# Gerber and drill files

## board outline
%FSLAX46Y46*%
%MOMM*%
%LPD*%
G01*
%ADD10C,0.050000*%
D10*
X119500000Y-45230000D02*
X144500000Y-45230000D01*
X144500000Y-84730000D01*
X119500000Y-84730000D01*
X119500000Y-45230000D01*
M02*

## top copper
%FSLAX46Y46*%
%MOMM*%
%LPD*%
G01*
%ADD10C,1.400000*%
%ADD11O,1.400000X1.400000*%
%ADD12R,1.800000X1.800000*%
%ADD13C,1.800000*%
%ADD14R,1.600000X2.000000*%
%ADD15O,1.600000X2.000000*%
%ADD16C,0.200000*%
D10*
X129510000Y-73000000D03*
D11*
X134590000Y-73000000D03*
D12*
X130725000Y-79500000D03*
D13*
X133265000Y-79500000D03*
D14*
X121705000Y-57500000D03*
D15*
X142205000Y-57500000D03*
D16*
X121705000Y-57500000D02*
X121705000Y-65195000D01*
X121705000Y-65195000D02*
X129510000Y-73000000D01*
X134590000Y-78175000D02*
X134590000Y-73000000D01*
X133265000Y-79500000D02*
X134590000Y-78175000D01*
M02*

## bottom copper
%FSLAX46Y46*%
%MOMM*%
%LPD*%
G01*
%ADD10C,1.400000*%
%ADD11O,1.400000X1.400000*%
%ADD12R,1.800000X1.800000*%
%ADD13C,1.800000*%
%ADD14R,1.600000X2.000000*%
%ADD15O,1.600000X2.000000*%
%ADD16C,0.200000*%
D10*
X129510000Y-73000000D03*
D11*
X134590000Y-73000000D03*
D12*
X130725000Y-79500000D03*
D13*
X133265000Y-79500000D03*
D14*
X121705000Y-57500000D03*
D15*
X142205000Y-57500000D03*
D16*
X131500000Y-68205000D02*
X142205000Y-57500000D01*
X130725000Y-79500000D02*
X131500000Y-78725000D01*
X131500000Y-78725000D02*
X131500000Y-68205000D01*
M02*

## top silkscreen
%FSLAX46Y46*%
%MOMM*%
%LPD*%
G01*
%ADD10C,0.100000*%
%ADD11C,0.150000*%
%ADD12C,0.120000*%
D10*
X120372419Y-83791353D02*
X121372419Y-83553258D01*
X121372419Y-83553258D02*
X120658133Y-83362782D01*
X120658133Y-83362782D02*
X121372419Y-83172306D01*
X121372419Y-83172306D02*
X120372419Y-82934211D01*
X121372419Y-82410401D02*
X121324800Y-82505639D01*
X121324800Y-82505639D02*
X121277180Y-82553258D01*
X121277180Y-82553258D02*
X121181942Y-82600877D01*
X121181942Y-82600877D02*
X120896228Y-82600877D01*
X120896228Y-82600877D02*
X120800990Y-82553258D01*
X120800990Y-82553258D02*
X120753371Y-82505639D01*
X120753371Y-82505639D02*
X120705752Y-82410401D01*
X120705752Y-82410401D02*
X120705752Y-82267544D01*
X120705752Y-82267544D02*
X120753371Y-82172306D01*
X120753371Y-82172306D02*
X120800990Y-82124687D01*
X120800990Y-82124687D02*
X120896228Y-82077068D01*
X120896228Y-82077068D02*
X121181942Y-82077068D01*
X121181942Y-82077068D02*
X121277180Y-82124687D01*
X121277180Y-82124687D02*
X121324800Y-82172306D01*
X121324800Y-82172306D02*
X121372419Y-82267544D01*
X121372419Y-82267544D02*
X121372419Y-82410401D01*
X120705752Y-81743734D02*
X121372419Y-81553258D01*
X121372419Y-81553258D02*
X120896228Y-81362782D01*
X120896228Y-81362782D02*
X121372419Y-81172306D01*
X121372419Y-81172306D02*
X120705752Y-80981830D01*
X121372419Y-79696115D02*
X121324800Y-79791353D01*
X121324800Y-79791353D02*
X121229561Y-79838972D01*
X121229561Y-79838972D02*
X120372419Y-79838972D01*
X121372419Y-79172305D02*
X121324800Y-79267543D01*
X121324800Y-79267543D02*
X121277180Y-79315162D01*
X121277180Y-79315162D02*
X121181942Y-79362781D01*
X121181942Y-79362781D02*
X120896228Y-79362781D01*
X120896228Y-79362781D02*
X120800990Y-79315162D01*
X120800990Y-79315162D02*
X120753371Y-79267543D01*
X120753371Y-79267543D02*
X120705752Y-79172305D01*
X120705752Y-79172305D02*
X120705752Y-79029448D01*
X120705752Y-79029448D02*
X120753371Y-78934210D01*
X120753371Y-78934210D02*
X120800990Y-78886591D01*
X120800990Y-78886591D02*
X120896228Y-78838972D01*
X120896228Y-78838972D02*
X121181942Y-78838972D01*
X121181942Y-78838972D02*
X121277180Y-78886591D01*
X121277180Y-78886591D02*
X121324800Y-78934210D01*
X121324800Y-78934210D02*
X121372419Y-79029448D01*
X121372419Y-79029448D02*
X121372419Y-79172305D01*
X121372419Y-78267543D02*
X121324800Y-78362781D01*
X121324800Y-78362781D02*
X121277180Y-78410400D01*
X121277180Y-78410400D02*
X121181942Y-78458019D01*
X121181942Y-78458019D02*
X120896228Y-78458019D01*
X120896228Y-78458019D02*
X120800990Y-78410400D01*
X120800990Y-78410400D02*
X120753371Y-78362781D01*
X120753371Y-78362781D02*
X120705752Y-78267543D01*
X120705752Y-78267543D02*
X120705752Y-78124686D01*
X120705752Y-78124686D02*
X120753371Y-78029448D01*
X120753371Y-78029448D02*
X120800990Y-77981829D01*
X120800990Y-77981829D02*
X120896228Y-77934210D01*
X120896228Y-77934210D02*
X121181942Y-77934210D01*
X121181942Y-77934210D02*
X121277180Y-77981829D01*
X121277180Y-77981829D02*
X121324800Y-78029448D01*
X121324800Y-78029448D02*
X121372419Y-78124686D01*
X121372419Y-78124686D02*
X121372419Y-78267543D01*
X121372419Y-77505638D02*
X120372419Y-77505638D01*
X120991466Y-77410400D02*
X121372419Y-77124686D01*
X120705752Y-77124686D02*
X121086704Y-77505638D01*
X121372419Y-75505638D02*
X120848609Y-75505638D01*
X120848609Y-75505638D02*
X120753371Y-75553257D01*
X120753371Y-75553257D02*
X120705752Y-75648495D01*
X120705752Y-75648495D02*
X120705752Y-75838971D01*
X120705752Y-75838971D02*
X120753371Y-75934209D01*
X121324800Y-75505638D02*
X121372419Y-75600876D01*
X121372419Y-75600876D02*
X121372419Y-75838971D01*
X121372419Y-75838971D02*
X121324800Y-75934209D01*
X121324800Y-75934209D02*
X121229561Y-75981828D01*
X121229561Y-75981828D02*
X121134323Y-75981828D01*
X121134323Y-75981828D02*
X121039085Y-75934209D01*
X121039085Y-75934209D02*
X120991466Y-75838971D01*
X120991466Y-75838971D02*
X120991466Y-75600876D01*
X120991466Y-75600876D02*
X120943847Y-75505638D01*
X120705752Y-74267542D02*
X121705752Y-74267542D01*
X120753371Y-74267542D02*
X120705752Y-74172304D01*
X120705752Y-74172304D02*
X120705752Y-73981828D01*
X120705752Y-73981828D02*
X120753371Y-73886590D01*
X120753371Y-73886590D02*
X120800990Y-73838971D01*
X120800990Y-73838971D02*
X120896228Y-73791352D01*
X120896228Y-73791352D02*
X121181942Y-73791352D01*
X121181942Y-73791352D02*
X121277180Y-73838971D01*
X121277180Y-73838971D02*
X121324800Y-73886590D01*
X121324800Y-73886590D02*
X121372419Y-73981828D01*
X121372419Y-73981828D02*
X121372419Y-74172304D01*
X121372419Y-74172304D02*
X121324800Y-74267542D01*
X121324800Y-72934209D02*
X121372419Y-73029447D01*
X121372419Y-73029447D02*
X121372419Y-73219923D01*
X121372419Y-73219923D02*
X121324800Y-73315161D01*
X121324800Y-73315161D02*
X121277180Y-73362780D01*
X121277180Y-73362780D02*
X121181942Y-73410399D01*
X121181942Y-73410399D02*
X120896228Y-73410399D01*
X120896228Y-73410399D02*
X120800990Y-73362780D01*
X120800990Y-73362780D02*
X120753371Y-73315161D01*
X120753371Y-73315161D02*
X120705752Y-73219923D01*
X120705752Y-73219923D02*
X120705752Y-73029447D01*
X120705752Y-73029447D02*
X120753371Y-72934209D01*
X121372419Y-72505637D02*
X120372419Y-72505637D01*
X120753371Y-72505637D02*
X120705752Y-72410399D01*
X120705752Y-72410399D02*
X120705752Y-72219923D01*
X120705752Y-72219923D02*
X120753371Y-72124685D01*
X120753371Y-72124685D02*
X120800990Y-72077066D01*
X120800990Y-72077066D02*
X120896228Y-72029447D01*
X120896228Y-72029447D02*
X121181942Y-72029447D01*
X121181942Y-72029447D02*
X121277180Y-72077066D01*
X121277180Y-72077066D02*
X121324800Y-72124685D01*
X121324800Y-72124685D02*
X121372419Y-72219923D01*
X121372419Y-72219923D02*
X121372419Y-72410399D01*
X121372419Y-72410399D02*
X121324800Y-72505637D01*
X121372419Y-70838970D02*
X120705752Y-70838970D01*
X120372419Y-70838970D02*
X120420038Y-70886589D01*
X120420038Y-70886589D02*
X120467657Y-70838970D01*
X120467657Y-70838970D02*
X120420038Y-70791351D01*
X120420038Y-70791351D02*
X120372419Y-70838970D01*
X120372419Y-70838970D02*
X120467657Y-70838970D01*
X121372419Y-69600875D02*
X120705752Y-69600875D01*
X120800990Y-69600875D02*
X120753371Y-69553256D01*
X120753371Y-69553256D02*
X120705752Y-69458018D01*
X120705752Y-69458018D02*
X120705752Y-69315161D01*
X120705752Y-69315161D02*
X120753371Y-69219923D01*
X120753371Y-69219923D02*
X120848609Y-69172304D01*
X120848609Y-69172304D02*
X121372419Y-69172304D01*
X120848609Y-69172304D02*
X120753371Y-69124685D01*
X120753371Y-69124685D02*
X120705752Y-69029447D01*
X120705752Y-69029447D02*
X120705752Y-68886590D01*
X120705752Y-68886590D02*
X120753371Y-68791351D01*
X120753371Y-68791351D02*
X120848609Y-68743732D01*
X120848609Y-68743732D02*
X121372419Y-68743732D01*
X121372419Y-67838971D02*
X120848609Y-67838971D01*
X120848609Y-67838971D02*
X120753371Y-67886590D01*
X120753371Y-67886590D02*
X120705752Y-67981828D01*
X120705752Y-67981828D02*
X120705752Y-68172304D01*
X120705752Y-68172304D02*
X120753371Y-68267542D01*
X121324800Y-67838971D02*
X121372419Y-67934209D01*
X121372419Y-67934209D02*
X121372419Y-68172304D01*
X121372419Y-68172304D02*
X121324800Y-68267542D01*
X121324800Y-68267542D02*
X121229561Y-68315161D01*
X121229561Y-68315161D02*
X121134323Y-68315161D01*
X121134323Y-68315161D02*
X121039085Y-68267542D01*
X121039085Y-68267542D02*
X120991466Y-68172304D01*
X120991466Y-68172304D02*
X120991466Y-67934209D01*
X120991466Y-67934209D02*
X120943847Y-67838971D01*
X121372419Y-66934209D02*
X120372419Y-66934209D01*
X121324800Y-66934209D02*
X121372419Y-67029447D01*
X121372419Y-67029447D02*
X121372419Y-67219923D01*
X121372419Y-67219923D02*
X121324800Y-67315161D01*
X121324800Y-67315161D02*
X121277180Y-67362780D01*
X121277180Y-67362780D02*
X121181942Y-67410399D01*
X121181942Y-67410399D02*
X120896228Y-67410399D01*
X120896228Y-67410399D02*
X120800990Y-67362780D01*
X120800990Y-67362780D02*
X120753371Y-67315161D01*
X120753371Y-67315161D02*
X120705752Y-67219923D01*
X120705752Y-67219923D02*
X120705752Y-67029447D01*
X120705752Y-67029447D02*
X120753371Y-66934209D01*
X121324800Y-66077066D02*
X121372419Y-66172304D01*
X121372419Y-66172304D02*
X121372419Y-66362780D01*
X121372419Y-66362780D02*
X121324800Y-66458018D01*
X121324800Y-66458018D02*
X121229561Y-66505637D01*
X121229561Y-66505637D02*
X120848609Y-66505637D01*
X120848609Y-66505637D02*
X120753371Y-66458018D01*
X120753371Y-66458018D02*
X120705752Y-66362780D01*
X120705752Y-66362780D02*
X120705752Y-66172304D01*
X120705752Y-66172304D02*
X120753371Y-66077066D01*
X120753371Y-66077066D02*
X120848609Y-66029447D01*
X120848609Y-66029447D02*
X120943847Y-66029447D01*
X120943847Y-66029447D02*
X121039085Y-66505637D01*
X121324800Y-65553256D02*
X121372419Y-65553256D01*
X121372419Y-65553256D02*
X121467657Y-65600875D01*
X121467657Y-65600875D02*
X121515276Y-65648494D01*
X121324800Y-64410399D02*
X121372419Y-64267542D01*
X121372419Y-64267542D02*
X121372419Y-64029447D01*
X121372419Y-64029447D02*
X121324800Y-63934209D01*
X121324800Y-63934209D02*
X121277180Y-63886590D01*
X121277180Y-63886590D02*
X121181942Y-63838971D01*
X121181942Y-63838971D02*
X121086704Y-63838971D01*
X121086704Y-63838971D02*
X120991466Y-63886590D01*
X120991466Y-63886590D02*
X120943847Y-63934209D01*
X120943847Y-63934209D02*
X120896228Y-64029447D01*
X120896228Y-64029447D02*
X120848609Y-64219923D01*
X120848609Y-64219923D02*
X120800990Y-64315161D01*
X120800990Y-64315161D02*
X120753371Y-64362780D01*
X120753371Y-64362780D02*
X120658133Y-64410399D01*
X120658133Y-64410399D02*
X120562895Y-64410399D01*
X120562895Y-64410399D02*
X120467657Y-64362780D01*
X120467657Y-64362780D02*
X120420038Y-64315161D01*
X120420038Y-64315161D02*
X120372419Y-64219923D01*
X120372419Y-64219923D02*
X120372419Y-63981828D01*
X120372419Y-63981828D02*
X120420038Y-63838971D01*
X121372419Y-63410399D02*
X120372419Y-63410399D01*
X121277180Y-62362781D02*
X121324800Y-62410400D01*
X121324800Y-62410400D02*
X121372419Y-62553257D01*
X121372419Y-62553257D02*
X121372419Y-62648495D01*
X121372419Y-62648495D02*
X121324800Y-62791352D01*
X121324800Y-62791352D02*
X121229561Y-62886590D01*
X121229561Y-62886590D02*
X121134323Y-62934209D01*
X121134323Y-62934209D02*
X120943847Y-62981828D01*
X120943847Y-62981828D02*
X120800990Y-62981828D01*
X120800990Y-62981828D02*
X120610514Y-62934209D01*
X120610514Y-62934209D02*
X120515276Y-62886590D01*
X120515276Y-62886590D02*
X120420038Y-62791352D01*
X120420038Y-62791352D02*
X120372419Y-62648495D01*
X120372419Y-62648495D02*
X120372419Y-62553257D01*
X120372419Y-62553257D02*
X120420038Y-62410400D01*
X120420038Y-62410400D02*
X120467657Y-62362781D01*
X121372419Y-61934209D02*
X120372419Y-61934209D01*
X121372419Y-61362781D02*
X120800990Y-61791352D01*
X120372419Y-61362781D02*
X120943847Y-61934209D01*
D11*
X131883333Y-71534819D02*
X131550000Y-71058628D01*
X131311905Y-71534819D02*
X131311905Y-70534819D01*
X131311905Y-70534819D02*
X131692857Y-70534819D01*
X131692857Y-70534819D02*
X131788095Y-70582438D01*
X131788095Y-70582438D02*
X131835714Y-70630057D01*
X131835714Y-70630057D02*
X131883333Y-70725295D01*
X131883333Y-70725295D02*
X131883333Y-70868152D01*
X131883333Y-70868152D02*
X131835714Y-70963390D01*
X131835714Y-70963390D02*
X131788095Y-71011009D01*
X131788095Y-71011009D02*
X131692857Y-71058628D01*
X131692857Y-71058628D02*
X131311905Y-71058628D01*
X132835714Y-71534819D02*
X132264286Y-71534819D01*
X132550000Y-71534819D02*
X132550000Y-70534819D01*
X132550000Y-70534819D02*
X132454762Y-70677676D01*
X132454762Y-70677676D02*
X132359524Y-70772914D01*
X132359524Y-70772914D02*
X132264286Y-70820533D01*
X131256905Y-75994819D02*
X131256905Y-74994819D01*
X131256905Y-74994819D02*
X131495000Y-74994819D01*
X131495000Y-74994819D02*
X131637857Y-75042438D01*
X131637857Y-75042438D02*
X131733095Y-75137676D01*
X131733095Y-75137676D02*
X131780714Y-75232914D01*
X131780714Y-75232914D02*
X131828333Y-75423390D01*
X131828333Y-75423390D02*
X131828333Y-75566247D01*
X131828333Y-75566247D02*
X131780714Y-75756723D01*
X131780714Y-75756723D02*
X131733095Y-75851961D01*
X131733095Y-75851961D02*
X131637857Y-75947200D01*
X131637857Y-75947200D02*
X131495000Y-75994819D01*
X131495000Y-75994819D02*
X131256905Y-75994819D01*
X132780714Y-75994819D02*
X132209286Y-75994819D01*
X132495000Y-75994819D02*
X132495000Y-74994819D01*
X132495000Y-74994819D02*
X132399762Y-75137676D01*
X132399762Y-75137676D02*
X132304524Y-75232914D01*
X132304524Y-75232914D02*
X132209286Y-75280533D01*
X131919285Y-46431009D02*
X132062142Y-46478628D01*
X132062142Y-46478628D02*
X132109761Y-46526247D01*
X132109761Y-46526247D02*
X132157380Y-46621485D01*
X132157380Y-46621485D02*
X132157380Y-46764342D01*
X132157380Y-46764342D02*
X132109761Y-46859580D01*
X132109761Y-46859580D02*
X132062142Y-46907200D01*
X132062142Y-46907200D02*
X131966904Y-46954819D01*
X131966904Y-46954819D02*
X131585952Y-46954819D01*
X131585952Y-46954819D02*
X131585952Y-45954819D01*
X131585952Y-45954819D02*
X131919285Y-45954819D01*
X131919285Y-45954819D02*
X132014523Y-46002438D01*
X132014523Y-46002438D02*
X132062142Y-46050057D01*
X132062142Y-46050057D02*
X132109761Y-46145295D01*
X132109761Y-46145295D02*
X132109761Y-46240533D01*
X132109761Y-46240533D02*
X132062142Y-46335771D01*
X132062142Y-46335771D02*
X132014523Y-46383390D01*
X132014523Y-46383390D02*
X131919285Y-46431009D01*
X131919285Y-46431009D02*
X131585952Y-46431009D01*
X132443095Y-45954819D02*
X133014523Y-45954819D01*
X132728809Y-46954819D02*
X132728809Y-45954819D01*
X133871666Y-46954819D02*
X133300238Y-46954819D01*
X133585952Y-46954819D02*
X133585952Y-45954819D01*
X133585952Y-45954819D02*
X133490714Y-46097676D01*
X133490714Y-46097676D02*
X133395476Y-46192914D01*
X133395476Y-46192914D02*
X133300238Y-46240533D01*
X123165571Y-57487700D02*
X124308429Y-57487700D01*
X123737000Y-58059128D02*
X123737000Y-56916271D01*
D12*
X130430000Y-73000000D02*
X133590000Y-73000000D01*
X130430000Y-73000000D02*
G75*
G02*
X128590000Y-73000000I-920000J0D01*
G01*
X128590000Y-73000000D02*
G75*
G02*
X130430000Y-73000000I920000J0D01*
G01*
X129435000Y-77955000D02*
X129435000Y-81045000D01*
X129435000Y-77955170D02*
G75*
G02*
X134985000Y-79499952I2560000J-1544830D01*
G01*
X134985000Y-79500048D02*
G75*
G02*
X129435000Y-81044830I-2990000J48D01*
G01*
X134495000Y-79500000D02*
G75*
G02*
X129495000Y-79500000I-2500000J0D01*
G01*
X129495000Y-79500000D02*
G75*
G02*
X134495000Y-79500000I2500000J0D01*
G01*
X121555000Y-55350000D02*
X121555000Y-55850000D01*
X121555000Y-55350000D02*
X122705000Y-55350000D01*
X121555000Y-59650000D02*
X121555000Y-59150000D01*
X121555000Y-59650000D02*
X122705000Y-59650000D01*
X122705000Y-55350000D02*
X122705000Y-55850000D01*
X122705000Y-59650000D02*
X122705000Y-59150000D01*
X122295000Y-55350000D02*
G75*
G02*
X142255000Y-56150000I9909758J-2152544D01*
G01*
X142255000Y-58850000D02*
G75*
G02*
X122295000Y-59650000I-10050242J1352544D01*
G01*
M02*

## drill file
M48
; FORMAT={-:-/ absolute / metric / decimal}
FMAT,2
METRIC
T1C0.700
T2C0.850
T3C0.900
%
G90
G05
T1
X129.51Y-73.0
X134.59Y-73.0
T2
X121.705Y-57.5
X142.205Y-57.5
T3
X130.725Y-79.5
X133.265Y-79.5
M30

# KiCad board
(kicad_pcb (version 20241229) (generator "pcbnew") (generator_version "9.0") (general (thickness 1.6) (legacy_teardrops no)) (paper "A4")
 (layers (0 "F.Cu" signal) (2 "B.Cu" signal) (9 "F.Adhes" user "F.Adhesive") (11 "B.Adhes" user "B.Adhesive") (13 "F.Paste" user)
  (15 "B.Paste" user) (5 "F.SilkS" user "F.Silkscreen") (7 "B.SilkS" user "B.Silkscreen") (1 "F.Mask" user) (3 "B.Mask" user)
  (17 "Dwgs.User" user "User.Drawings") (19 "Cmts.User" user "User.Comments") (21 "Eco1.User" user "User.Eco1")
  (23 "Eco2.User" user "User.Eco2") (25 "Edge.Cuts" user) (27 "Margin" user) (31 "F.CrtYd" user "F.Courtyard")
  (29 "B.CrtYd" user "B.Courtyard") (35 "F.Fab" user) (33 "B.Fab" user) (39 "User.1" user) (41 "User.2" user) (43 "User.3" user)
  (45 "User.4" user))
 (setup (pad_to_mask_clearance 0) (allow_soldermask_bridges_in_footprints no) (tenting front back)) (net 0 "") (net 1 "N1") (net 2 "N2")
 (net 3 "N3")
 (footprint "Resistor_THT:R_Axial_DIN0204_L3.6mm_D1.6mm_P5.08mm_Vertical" (layer "F.Cu") (at 129.51 73)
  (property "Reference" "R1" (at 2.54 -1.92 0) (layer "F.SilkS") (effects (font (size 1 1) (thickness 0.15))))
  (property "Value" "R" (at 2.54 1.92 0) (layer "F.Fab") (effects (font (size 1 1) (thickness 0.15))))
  (fp_line (start 0.92 0) (end 4.08 0) (stroke (width 0.12) (type solid)) (layer "F.SilkS"))
  (fp_circle (center 0 0) (end 0.92 0) (stroke (width 0.12) (type solid)) (fill no) (layer "F.SilkS"))
  (pad "1" thru_hole circle (at 0 0) (size 1.4 1.4) (drill 0.7) (layers "*.Cu" "*.Mask") (remove_unused_layers no) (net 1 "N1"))
  (pad "2" thru_hole oval (at 5.08 0) (size 1.4 1.4) (drill 0.7) (layers "*.Cu" "*.Mask") (remove_unused_layers no) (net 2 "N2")))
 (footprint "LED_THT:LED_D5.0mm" (layer "F.Cu") (at 130.725 79.5)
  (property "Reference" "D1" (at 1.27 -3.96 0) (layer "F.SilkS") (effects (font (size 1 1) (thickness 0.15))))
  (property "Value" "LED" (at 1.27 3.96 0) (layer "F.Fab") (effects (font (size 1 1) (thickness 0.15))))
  (fp_line (start -1.29 -1.545) (end -1.29 1.545) (stroke (width 0.12) (type solid)) (layer "F.SilkS"))
  (fp_arc (start -1.29 -1.54483) (mid 2.071756 -2.880501) (end 4.26 -0.000048) (stroke (width 0.12) (type solid)) (layer "F.SilkS"))
  (fp_arc (start 4.26 0.000048) (mid 2.071756 2.880501) (end -1.29 1.54483) (stroke (width 0.12) (type solid)) (layer "F.SilkS"))
  (fp_circle (center 1.27 0) (end 3.77 0) (stroke (width 0.12) (type solid)) (fill no) (layer "F.SilkS"))
  (pad "1" thru_hole rect (at 0 0) (size 1.8 1.8) (drill 0.9) (layers "*.Cu" "*.Mask") (remove_unused_layers no) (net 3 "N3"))
  (pad "2" thru_hole circle (at 2.54 0) (size 1.8 1.8) (drill 0.9) (layers "*.Cu" "*.Mask") (remove_unused_layers no) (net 2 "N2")))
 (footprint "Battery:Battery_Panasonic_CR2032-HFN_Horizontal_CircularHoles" (layer "F.Cu") (at 121.705 57.5)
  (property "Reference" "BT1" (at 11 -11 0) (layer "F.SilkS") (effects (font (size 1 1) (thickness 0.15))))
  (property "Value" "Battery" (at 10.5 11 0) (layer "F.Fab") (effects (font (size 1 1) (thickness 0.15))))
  (fp_line (start -0.15 -2.15) (end -0.15 -1.65) (stroke (width 0.12) (type default)) (layer "F.SilkS"))
  (fp_line (start -0.15 -2.15) (end 1 -2.15) (stroke (width 0.12) (type default)) (layer "F.SilkS"))
  (fp_line (start -0.15 2.15) (end -0.15 1.65) (stroke (width 0.12) (type default)) (layer "F.SilkS"))
  (fp_line (start -0.15 2.15) (end 1 2.15) (stroke (width 0.12) (type default)) (layer "F.SilkS"))
  (fp_line (start 1 -2.15) (end 1 -1.65) (stroke (width 0.12) (type default)) (layer "F.SilkS"))
  (fp_line (start 1 2.15) (end 1 1.65) (stroke (width 0.12) (type default)) (layer "F.SilkS"))
  (fp_arc (start 0.59 -2.15) (mid 10.91 -10.13) (end 20.55 -1.35) (stroke (width 0.12) (type default)) (layer "F.SilkS"))
  (fp_arc (start 20.55 1.35) (mid 10.91 10.13) (end 0.59 2.15) (stroke (width 0.12) (type default)) (layer "F.SilkS"))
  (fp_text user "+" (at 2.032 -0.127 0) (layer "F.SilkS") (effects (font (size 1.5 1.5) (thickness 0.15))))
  (pad "1" thru_hole rect (at 0 0) (size 1.6 2) (drill 0.85) (layers "*.Cu" "*.Mask") (remove_unused_layers no) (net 1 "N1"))
  (pad "2" thru_hole oval (at 20.5 0) (size 1.6 2) (drill 0.85) (layers "*.Cu" "*.Mask") (remove_unused_layers no) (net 3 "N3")))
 (gr_rect (start 119.5 45.23) (end 144.5 84.73) (stroke (width 0.05) (type default)) (fill no) (layer "Edge.Cuts"))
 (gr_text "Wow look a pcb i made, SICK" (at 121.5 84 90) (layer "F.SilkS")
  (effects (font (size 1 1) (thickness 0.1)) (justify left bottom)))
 (segment (start 121.705 57.5) (end 121.705 65.195) (width 0.2) (layer "F.Cu") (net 1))
 (segment (start 121.705 65.195) (end 129.51 73) (width 0.2) (layer "F.Cu") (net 1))
 (segment (start 131.5 68.205) (end 142.205 57.5) (width 0.2) (layer "B.Cu") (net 3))
 (segment (start 130.725 79.5) (end 131.5 78.725) (width 0.2) (layer "B.Cu") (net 3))
 (segment (start 131.5 78.725) (end 131.5 68.205) (width 0.2) (layer "B.Cu") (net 3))
 (segment (start 134.59 78.175) (end 134.59 73) (width 0.2) (layer "F.Cu") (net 2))
 (segment (start 133.265 79.5) (end 134.59 78.175) (width 0.2) (layer "F.Cu") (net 2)))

